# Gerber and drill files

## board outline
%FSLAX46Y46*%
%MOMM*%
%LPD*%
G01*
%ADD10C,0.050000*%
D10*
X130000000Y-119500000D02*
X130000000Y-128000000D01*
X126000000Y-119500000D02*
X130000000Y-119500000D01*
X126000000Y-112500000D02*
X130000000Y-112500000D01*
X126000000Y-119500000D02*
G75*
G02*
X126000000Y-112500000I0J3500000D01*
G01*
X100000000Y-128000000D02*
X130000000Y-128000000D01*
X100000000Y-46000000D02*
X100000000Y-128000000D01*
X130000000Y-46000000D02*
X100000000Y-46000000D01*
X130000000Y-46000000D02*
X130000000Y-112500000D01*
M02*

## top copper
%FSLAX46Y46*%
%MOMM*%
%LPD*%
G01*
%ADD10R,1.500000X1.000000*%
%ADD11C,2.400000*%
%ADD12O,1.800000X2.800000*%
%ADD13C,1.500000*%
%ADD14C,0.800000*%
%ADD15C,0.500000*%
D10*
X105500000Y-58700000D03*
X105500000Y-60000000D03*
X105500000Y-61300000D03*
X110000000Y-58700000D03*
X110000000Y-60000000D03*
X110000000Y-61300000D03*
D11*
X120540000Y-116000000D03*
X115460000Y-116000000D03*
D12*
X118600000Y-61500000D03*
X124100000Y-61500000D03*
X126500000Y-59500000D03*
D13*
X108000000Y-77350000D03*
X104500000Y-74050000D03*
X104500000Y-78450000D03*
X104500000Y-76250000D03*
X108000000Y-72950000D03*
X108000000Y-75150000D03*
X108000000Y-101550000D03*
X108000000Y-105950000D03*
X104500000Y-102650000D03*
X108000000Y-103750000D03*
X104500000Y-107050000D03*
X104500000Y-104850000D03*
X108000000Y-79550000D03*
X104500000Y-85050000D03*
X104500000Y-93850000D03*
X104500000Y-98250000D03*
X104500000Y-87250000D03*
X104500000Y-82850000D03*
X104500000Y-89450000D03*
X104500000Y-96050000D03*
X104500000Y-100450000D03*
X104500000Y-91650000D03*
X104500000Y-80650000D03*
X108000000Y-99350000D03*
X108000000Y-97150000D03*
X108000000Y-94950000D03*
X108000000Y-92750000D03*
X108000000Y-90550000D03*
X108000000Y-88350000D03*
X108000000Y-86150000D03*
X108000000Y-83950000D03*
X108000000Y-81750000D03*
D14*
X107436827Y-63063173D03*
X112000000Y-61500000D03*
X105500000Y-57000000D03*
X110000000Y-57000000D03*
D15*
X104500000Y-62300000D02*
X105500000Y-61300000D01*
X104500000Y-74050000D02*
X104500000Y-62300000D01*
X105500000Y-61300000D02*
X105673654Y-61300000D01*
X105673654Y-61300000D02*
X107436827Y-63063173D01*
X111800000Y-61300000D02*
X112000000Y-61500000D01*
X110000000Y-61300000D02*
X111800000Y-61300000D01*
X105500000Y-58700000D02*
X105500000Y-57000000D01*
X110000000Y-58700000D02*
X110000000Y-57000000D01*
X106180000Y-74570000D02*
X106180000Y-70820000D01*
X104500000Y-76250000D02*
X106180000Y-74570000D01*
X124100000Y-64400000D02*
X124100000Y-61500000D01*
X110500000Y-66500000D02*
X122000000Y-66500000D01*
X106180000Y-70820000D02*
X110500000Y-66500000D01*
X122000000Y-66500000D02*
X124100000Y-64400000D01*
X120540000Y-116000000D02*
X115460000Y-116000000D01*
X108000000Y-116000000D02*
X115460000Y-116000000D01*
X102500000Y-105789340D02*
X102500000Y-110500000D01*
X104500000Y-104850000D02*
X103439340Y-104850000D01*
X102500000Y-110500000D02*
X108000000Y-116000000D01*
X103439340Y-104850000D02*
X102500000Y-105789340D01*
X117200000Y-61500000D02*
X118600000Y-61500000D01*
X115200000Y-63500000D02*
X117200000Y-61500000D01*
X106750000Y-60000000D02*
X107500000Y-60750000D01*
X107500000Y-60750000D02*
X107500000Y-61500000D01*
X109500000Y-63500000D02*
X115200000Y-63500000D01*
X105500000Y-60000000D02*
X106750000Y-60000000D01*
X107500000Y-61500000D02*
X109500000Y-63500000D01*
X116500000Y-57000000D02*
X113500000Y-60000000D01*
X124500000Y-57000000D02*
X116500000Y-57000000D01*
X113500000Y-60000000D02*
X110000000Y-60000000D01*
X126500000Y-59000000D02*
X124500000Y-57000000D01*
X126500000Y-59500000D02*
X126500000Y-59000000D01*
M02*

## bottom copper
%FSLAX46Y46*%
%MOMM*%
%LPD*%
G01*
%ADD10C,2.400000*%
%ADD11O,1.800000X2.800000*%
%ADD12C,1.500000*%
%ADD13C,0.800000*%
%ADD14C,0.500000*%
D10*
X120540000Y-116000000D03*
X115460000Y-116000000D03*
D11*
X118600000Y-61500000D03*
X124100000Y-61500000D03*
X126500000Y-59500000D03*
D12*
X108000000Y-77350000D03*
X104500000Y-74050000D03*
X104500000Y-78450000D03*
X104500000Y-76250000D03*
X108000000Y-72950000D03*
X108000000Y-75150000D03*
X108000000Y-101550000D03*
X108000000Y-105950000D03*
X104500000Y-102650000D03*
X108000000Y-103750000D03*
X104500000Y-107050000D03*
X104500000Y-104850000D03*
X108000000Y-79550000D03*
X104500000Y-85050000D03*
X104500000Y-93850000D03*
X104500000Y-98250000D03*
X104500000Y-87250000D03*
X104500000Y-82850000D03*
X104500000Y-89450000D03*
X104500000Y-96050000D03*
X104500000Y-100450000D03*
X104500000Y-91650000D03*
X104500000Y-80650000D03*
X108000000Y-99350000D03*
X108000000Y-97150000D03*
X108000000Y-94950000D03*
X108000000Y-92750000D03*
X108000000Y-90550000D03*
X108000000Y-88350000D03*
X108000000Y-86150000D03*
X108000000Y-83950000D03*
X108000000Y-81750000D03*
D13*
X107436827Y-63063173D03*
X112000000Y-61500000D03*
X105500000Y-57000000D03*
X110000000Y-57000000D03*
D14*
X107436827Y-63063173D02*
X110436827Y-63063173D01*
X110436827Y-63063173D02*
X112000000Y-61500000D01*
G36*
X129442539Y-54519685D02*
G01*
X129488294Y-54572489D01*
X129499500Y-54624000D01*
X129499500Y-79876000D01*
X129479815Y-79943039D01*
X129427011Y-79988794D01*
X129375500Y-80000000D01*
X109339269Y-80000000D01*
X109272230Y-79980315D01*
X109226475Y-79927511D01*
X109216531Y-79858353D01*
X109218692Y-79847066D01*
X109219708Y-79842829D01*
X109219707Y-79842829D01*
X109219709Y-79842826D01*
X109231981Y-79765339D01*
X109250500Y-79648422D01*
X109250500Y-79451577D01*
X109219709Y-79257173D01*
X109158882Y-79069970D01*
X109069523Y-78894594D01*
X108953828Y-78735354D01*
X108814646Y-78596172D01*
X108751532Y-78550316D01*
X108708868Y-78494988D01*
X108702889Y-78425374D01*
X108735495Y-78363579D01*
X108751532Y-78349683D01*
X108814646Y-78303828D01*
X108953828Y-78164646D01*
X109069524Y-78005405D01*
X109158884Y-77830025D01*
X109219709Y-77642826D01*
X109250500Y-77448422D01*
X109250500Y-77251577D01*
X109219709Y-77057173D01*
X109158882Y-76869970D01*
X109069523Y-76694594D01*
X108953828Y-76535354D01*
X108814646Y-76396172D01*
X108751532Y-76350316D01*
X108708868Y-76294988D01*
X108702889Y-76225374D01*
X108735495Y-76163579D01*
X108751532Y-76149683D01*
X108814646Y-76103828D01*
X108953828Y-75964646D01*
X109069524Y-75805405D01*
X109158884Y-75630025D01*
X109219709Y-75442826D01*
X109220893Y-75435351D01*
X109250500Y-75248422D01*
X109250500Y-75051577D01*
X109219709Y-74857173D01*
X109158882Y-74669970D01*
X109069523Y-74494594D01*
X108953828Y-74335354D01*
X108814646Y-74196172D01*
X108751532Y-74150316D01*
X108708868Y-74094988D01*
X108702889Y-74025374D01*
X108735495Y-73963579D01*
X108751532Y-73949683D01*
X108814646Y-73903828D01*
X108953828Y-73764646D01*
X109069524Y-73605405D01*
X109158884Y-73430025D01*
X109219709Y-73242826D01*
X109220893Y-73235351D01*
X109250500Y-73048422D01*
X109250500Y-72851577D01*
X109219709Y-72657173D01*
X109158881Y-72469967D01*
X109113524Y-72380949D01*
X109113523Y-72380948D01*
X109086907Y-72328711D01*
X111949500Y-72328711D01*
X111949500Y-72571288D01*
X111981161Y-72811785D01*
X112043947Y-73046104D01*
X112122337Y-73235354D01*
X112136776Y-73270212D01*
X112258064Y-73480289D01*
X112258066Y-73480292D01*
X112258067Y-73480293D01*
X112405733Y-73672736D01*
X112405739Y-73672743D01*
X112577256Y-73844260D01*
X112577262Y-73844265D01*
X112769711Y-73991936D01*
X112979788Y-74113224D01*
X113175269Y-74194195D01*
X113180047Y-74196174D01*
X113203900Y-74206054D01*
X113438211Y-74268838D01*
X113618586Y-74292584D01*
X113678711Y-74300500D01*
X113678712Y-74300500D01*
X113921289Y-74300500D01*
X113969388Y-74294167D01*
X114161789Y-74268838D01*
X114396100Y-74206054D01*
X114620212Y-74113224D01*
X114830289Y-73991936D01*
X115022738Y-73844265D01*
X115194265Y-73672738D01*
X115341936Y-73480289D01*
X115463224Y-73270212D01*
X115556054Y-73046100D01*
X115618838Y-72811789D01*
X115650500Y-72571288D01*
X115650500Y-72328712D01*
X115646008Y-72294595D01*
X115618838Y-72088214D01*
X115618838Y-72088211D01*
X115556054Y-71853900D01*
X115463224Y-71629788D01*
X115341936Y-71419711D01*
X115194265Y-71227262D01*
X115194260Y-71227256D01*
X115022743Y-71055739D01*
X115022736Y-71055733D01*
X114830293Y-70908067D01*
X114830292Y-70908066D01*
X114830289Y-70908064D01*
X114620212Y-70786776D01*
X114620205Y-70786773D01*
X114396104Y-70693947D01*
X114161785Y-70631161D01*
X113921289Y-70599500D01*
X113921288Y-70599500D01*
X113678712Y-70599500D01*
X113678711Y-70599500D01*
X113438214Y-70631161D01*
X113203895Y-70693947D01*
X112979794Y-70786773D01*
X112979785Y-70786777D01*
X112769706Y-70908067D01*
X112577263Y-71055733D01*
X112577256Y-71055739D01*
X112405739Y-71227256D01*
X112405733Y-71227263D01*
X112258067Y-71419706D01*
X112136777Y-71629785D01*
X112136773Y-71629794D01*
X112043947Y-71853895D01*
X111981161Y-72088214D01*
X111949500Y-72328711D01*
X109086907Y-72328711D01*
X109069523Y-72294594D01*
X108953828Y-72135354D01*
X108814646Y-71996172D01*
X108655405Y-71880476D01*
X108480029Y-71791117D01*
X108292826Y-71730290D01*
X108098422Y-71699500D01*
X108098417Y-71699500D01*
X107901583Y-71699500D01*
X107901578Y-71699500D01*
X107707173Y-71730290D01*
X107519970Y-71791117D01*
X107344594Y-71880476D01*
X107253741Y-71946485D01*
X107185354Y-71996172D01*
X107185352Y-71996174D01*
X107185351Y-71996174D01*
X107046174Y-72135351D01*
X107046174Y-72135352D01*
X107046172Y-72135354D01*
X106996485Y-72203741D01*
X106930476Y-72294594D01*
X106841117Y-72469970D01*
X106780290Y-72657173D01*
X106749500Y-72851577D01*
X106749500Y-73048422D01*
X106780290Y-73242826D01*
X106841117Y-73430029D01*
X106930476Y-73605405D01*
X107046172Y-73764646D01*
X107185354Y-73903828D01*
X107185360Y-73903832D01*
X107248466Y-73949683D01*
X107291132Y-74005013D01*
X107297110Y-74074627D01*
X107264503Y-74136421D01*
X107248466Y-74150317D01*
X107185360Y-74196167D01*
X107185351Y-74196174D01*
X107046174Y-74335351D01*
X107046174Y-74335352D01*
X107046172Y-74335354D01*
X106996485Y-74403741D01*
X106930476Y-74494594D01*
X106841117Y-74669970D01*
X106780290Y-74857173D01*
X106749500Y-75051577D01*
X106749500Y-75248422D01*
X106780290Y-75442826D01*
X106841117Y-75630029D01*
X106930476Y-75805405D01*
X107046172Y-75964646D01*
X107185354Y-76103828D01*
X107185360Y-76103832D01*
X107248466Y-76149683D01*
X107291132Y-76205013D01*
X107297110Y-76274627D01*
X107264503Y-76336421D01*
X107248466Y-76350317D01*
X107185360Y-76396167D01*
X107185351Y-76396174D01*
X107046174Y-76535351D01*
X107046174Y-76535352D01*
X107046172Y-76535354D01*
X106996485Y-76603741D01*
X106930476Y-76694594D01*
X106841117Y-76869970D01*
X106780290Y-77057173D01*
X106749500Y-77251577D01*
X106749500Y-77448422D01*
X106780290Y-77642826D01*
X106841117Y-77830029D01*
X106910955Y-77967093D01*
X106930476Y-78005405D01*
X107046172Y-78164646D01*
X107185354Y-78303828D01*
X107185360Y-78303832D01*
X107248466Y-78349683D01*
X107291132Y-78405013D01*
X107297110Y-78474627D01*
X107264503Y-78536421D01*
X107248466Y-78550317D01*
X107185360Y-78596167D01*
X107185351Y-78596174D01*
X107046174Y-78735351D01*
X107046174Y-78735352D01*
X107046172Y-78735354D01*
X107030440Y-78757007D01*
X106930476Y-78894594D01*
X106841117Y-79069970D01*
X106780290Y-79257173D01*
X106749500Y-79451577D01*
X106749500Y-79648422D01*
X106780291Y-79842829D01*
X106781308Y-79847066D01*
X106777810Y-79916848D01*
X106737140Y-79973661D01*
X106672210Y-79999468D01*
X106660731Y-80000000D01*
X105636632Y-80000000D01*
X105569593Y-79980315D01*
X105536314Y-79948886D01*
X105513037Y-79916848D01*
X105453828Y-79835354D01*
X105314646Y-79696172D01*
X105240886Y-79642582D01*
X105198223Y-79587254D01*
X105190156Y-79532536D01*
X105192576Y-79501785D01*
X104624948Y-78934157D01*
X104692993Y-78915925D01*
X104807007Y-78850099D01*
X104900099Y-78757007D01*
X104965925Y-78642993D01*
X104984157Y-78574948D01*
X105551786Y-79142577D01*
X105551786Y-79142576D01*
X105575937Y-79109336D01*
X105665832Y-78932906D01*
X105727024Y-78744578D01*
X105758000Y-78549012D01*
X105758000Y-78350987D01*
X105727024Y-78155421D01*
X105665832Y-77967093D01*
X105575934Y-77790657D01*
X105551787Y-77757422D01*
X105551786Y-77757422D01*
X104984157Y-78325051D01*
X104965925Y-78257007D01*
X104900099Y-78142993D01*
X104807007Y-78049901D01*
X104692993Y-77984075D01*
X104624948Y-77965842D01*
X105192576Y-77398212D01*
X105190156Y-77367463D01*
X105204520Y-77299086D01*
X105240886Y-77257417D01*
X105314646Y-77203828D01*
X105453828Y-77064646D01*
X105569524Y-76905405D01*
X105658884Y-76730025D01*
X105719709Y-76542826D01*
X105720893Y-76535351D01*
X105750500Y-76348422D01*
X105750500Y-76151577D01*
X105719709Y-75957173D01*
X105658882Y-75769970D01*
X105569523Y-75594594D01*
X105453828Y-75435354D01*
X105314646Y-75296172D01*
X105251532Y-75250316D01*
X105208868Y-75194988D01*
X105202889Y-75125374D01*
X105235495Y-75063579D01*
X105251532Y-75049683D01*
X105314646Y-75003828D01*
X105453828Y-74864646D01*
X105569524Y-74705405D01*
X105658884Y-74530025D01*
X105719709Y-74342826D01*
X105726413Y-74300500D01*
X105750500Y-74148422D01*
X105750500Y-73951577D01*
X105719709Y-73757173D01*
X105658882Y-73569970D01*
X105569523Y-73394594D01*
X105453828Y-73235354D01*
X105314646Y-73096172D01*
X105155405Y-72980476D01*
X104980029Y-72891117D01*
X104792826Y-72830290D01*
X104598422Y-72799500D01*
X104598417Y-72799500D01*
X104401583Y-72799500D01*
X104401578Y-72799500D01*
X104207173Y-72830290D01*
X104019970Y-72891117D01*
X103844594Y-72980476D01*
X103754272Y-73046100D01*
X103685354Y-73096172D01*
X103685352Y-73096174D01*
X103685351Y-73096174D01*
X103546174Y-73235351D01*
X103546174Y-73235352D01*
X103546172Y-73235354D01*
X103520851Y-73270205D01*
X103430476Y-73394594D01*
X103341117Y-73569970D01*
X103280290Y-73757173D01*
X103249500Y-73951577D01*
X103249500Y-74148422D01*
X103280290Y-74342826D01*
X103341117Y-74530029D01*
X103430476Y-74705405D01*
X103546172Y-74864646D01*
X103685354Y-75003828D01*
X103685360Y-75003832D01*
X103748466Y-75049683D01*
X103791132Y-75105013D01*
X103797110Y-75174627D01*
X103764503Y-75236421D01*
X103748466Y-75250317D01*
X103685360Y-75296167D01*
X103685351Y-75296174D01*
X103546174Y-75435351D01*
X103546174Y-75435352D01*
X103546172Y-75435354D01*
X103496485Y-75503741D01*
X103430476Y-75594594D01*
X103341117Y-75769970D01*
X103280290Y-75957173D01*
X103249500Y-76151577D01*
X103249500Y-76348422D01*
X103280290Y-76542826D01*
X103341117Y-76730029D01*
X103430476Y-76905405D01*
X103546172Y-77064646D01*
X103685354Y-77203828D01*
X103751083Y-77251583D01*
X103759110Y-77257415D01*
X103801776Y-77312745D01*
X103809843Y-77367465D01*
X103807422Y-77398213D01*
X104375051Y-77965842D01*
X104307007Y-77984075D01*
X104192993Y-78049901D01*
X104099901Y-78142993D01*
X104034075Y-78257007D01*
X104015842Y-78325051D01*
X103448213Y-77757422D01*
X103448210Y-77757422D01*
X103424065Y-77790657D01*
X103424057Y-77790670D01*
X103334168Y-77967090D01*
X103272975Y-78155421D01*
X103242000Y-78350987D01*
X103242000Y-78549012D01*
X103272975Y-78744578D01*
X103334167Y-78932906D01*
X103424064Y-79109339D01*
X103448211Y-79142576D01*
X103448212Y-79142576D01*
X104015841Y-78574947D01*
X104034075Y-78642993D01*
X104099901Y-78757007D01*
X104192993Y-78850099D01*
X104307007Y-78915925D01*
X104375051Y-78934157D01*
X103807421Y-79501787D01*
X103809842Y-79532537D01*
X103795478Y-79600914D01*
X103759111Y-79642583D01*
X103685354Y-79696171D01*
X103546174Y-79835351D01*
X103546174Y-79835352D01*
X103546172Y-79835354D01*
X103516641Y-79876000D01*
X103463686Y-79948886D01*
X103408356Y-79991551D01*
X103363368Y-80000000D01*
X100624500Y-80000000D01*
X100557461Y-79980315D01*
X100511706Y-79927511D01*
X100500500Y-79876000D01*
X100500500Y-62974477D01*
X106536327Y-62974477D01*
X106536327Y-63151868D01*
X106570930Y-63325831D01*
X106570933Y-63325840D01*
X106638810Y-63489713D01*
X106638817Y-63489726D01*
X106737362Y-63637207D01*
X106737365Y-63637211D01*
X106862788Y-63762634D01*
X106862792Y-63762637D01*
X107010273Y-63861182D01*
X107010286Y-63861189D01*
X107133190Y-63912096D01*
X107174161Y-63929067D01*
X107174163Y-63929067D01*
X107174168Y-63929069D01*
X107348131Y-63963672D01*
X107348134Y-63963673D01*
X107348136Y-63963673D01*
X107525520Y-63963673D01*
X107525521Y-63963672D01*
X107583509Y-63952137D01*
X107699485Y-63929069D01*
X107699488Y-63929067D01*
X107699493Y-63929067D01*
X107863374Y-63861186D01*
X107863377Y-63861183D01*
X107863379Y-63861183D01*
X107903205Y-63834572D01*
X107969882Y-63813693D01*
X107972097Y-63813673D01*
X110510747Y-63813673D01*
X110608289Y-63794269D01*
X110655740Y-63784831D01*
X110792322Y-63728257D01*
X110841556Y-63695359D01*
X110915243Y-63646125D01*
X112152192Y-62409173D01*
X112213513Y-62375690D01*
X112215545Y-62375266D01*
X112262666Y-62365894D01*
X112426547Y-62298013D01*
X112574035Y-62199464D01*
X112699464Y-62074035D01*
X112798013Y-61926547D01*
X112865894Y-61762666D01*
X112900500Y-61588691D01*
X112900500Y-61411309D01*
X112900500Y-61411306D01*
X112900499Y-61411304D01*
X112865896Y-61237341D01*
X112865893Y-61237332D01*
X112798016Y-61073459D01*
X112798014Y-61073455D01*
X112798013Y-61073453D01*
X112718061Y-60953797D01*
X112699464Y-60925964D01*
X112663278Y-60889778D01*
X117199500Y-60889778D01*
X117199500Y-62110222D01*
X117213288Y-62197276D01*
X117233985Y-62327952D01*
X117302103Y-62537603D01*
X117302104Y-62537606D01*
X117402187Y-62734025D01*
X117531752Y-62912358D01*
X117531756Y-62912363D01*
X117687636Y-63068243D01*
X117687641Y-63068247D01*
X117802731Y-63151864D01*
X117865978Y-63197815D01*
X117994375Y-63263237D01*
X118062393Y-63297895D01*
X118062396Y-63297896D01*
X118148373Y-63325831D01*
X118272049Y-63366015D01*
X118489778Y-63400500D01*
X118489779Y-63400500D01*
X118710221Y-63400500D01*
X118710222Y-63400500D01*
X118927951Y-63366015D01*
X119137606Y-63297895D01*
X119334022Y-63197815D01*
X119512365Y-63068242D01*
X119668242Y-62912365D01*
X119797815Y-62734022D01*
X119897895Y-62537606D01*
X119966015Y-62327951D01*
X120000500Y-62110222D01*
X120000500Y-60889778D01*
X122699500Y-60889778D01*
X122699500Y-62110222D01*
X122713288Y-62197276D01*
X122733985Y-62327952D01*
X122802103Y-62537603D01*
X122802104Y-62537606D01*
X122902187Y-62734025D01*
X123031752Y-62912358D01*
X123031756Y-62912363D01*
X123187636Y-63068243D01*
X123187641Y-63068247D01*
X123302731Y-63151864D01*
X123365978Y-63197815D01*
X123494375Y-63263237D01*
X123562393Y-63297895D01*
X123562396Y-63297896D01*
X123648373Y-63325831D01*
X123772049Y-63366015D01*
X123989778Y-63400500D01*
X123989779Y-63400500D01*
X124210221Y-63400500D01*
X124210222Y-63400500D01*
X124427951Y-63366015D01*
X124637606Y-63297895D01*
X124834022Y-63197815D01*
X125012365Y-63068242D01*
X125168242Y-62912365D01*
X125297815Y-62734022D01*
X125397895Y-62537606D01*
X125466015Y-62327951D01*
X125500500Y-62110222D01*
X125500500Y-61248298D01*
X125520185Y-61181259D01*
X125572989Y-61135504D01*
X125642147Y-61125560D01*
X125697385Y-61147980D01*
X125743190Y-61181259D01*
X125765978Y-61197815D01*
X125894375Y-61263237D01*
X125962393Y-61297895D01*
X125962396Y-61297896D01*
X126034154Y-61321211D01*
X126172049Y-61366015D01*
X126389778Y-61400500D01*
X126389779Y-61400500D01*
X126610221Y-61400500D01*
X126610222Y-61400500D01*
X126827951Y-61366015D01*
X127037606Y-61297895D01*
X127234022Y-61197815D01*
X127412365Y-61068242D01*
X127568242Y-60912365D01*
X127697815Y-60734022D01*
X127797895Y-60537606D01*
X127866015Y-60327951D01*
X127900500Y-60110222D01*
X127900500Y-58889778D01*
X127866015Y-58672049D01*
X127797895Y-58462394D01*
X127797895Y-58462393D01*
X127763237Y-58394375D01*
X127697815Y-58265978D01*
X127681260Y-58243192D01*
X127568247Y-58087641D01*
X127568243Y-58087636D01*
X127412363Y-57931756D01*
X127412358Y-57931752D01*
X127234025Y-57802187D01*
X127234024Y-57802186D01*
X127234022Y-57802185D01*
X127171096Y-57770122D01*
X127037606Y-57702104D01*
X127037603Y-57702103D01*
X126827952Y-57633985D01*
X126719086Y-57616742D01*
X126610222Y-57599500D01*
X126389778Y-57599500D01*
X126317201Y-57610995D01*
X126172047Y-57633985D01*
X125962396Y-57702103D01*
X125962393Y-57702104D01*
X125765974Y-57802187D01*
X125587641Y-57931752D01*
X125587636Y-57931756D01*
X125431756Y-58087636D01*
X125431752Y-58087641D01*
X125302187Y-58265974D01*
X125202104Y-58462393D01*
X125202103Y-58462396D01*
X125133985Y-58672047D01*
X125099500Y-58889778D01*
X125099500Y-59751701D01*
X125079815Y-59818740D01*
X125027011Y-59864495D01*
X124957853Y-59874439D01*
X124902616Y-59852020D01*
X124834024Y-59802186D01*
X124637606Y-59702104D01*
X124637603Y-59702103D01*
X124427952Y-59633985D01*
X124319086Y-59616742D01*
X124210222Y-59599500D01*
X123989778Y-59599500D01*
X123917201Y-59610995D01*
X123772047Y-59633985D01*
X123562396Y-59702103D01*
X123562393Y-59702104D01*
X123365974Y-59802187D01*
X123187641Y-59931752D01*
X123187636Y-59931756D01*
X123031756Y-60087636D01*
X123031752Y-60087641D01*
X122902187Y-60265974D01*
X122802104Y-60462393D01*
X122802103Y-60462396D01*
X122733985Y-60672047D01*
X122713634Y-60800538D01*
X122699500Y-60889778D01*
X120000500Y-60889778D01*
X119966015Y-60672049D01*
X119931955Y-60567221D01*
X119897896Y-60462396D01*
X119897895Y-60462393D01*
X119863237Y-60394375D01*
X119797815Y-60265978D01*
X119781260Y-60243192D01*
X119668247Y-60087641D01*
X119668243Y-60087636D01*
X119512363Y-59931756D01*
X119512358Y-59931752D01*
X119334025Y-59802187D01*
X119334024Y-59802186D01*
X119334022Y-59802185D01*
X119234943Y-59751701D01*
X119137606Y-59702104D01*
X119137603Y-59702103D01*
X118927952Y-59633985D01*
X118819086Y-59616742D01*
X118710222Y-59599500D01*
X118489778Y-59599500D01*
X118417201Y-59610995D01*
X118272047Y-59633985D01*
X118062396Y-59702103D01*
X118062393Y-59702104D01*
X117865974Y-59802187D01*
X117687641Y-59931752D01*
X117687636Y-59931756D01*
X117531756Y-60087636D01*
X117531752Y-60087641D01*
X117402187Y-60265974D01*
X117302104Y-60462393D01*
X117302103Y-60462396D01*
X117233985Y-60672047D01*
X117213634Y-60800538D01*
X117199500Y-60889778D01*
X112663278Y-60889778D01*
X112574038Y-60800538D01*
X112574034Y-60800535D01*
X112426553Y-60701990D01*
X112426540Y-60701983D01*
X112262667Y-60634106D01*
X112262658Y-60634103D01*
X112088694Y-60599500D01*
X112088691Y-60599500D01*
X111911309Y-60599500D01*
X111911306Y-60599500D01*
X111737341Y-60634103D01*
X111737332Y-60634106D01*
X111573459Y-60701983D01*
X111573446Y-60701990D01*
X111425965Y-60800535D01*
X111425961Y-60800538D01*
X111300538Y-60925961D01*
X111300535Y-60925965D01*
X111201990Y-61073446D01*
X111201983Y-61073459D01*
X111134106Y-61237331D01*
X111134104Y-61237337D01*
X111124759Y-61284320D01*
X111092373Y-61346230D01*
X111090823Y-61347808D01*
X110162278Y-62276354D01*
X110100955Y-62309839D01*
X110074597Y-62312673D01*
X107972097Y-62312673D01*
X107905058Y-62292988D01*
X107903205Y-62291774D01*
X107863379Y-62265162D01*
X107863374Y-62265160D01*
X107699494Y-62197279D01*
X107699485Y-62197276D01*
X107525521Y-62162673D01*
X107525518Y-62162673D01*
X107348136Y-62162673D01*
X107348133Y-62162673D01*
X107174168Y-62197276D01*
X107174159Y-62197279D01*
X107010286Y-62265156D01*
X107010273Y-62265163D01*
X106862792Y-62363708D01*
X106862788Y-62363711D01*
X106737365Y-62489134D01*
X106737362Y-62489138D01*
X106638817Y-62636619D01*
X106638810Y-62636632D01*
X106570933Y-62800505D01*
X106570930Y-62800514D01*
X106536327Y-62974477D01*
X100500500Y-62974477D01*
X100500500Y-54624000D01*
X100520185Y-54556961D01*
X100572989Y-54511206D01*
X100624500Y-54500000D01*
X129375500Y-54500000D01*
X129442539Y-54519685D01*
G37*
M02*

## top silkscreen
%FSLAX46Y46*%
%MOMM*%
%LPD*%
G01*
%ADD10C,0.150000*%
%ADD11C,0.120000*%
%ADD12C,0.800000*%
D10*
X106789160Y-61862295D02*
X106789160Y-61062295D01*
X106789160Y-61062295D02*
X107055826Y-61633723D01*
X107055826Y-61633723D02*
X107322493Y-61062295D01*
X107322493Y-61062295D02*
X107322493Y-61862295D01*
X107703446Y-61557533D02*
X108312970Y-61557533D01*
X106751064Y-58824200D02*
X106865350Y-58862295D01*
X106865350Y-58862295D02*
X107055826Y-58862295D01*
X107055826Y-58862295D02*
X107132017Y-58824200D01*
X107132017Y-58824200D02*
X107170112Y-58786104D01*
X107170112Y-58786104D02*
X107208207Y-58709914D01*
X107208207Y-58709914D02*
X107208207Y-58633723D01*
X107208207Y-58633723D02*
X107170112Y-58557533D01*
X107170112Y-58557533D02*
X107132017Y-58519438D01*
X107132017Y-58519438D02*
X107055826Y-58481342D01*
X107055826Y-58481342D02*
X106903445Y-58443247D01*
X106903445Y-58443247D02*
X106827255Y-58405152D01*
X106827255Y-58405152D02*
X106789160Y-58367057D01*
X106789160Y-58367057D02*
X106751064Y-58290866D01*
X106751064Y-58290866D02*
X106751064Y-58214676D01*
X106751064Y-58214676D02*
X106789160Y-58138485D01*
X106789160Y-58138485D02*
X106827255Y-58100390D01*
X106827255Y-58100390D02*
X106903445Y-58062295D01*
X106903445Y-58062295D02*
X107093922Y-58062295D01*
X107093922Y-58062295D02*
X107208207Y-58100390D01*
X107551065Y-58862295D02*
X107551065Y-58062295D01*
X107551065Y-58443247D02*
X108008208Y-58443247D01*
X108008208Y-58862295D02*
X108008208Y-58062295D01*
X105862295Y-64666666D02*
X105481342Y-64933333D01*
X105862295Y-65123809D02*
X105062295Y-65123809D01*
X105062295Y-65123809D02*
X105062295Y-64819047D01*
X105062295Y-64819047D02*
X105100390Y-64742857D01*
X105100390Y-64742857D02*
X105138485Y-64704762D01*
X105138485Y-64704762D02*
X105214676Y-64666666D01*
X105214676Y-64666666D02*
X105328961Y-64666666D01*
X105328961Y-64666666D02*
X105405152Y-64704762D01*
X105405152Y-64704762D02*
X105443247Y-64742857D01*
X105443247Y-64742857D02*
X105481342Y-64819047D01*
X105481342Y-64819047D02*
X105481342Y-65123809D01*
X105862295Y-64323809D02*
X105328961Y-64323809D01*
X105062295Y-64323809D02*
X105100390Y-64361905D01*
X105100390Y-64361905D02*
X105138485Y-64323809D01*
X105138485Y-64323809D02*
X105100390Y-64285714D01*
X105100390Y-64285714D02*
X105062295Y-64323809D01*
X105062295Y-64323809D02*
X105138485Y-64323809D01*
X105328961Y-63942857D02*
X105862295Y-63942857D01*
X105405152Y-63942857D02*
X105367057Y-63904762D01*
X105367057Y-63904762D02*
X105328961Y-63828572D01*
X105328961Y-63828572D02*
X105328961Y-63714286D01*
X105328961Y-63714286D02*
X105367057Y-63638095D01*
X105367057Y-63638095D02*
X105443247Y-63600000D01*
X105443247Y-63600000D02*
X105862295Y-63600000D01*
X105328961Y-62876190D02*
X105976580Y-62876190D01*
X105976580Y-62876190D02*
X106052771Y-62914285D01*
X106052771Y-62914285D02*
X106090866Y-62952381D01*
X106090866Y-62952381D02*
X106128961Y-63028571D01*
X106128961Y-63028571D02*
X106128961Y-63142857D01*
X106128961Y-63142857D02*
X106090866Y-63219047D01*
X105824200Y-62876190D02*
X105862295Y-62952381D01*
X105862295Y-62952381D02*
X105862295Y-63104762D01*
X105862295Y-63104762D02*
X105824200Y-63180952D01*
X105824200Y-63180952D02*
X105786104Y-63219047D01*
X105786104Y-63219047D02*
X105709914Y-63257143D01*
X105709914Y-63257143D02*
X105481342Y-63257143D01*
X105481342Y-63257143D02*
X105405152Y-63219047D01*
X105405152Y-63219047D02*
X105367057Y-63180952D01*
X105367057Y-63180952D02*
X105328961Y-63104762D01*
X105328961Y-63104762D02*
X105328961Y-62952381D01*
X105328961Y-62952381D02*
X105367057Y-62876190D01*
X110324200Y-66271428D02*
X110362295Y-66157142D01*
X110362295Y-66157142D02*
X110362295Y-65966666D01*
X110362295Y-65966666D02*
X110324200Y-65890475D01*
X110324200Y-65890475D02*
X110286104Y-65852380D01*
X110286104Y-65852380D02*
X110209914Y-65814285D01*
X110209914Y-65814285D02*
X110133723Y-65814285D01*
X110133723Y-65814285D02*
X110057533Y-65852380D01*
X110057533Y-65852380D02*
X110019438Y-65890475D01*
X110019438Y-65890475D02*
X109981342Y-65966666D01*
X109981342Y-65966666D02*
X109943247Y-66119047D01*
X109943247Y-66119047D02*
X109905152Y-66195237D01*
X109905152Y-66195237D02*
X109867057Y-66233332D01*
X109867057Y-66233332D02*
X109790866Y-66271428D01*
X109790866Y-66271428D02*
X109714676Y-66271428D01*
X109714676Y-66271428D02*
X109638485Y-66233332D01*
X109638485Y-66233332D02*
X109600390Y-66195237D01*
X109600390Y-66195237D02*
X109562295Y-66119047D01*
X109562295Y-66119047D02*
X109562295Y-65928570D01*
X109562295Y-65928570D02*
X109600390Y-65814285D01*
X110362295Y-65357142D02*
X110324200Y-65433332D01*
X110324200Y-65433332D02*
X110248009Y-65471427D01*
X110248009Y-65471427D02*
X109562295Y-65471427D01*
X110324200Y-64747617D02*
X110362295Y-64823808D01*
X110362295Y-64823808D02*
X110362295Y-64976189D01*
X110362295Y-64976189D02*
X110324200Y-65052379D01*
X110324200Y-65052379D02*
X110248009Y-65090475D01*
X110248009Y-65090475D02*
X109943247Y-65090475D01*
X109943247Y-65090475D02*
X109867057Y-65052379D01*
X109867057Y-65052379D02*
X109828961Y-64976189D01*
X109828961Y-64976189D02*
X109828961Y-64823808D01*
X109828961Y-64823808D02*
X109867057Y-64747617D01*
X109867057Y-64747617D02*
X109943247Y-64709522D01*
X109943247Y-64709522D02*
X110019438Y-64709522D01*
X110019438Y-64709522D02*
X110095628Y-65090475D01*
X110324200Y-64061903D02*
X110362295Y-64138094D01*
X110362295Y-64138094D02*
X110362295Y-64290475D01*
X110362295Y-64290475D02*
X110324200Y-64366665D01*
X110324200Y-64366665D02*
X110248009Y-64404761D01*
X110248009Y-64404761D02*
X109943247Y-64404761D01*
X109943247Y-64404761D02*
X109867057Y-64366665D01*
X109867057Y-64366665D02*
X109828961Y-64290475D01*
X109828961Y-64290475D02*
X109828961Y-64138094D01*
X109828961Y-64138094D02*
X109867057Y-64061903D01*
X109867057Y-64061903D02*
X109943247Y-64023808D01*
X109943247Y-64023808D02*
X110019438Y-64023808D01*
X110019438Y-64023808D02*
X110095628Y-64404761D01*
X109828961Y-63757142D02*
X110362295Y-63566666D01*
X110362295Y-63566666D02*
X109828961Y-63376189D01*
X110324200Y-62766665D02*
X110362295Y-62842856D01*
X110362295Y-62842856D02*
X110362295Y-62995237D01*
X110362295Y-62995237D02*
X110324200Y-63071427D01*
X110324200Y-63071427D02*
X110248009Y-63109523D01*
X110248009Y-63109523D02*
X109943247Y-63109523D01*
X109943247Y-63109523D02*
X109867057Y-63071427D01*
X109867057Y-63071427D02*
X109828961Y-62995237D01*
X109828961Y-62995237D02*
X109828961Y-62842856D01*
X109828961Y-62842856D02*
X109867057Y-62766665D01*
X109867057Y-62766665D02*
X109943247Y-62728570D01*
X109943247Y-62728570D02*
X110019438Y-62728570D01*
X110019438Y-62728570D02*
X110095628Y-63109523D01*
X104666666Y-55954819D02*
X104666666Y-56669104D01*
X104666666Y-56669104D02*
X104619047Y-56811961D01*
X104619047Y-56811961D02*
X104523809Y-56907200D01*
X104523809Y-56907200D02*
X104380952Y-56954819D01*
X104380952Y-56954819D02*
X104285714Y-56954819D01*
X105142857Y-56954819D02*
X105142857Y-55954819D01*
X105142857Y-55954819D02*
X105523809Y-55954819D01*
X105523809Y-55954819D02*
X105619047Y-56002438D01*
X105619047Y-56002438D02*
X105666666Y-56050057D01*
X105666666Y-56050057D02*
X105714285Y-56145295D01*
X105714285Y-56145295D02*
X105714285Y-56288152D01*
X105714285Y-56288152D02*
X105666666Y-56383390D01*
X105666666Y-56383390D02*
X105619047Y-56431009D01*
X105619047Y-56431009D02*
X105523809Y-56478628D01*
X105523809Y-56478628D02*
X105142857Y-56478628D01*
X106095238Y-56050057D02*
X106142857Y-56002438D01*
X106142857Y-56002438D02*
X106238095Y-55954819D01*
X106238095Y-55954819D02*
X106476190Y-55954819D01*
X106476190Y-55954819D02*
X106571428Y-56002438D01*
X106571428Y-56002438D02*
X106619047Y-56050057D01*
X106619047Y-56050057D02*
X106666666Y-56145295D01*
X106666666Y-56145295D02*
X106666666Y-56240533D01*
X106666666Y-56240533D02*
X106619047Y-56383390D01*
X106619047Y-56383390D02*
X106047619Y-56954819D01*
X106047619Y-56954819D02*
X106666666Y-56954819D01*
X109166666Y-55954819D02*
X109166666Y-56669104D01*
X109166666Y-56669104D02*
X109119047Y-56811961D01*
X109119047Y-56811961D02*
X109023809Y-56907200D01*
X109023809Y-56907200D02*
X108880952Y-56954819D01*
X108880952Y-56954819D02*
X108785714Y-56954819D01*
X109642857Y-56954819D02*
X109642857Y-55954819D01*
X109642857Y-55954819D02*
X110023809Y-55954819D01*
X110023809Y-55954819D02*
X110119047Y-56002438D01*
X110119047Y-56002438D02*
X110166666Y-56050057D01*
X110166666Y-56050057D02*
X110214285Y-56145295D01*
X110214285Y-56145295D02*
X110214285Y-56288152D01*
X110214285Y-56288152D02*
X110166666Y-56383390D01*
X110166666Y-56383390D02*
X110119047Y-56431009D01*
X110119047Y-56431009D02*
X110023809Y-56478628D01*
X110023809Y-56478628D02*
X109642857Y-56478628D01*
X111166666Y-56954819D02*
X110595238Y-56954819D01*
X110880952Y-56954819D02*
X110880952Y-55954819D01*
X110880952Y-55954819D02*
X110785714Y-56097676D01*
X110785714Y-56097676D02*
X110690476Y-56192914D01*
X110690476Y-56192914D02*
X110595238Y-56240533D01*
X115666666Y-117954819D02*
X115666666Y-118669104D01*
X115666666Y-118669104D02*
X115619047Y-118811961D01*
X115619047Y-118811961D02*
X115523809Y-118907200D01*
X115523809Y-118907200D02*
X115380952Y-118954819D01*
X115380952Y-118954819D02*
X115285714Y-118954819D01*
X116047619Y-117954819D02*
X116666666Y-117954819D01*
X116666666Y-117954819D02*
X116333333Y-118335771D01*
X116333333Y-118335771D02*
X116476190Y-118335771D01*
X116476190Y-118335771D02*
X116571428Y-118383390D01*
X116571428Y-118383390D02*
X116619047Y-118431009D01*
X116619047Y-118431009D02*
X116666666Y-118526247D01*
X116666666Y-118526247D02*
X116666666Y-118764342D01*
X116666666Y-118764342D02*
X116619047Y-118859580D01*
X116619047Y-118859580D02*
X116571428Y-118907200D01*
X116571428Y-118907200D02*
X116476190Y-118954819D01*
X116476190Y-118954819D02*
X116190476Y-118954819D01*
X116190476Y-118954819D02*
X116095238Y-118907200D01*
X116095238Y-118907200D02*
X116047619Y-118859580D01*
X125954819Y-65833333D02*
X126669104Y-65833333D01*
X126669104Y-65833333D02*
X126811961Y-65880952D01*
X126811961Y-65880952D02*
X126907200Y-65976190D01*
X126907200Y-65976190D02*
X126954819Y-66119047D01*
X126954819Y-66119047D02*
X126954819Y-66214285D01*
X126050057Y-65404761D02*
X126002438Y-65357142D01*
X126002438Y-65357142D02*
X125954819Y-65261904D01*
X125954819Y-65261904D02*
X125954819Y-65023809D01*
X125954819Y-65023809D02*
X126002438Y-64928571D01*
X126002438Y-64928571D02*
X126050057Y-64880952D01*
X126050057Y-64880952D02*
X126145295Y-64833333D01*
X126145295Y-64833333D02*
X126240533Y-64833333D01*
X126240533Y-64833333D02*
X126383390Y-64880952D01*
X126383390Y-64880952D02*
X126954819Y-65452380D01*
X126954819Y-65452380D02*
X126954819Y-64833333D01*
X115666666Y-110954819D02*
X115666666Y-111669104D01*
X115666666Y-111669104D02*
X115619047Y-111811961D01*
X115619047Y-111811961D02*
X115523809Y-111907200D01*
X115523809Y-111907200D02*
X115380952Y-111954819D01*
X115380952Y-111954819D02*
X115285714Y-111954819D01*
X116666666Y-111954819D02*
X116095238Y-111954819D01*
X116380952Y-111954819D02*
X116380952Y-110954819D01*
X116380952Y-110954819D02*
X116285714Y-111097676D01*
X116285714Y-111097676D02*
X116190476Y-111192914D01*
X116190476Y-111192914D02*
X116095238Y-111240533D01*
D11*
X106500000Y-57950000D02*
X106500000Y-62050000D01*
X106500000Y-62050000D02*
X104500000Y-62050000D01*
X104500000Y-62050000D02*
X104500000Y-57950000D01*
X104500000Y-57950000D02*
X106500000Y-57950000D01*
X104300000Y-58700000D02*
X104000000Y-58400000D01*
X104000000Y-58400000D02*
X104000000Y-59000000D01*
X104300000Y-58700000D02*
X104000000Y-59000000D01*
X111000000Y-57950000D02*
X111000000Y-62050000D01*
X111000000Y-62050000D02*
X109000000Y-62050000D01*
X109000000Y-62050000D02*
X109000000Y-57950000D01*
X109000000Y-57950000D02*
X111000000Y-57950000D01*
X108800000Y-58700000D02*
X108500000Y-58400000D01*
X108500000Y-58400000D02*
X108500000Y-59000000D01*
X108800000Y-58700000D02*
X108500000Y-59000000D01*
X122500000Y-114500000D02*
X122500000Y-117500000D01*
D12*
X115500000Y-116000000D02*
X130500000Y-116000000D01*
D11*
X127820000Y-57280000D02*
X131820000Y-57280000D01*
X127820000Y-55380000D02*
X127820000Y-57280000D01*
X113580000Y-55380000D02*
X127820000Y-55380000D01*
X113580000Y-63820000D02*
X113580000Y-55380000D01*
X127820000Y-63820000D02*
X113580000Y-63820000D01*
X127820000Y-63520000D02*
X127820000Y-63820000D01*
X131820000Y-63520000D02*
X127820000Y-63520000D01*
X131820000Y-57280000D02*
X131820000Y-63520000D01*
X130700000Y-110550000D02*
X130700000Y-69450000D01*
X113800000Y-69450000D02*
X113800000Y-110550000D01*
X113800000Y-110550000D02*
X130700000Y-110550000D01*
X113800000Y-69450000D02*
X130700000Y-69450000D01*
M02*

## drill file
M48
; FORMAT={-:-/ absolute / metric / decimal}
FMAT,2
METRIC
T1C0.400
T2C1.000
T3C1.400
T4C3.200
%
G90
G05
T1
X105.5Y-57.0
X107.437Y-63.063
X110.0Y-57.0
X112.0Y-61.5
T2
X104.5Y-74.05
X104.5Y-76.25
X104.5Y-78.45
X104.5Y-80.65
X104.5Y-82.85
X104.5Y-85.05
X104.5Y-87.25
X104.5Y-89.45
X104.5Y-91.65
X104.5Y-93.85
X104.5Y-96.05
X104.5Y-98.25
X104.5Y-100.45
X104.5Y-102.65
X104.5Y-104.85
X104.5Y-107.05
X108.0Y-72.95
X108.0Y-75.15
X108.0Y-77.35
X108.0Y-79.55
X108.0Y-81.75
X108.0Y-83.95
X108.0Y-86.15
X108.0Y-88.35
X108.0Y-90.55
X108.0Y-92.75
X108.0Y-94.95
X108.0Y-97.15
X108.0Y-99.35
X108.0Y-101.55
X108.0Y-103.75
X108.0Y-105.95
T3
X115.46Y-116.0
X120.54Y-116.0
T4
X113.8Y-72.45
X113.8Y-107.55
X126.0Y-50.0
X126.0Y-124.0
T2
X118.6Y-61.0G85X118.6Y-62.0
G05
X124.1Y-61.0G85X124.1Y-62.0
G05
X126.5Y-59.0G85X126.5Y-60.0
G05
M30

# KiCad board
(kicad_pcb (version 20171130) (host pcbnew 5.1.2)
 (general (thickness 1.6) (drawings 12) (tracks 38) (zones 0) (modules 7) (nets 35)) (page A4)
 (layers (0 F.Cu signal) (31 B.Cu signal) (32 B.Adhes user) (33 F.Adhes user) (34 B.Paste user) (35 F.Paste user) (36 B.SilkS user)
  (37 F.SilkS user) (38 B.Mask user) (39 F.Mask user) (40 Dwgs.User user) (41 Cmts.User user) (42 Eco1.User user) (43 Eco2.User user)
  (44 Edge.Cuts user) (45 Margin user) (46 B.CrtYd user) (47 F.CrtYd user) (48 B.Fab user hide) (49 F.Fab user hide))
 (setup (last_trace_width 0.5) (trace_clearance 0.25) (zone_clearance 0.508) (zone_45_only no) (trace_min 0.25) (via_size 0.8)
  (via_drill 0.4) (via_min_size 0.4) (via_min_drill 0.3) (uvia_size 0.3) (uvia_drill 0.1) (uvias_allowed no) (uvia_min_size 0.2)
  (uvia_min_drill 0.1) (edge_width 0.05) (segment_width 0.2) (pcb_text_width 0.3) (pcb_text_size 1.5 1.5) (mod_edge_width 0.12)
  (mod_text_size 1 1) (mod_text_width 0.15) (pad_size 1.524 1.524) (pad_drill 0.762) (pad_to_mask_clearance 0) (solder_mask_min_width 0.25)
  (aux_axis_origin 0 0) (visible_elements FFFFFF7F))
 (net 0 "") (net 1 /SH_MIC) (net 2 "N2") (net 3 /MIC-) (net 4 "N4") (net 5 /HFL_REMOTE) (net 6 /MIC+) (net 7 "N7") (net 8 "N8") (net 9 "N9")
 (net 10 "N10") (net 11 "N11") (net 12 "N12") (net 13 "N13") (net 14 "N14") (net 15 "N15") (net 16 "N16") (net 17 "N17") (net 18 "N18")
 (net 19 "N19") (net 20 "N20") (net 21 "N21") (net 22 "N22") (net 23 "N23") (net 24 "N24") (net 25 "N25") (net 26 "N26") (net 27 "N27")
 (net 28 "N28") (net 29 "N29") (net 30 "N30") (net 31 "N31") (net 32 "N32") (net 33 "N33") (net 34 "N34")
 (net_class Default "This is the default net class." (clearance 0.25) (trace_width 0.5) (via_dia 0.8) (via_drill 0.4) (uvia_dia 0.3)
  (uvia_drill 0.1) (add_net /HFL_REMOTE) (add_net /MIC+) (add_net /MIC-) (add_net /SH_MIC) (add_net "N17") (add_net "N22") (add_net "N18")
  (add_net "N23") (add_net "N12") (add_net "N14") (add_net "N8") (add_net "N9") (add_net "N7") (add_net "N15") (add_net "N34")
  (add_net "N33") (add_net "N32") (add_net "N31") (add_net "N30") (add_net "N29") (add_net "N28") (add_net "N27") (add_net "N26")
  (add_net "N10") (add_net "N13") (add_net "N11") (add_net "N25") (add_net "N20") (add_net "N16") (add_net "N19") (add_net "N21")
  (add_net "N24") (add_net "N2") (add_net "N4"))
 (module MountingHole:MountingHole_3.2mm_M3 (layer F.Cu) (at 126 124)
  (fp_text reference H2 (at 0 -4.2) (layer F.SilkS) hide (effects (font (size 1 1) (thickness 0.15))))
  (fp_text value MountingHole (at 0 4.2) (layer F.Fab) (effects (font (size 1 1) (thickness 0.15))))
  (pad 1 np_thru_hole circle (at 0 0) (size 3.2 3.2) (drill 3.2) (layers *.Cu *.Mask)))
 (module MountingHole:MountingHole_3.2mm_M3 (layer F.Cu) (at 126 50)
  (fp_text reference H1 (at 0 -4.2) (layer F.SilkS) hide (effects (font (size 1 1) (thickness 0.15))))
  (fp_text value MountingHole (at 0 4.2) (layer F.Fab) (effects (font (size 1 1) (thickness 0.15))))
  (pad 1 np_thru_hole circle (at 0 0) (size 3.2 3.2) (drill 3.2) (layers *.Cu *.Mask)))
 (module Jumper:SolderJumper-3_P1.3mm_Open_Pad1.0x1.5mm (layer F.Cu) (at 105.5 60 270)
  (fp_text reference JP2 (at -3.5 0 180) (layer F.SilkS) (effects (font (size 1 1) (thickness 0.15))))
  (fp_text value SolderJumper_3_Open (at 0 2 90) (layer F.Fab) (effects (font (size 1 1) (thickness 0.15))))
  (fp_line (start -2.05 -1) (end 2.05 -1) (layer F.SilkS) (width 0.12))
  (fp_line (start 2.05 -1) (end 2.05 1) (layer F.SilkS) (width 0.12))
  (fp_line (start 2.05 1) (end -2.05 1) (layer F.SilkS) (width 0.12))
  (fp_line (start -2.05 1) (end -2.05 -1) (layer F.SilkS) (width 0.12))
  (fp_line (start -1.3 1.2) (end -1.6 1.5) (layer F.SilkS) (width 0.12))
  (fp_line (start -1.6 1.5) (end -1 1.5) (layer F.SilkS) (width 0.12))
  (fp_line (start -1.3 1.2) (end -1 1.5) (layer F.SilkS) (width 0.12))
  (pad 1 smd rect (at -1.3 0 270) (size 1 1.5) (layers F.Cu F.Mask) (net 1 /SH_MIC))
  (pad 2 smd rect (at 0 0 270) (size 1 1.5) (layers F.Cu F.Mask) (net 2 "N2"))
  (pad 3 smd rect (at 1.3 0 270) (size 1 1.5) (layers F.Cu F.Mask) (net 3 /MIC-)))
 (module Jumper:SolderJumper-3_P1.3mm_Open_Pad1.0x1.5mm (layer F.Cu) (at 110 60 270)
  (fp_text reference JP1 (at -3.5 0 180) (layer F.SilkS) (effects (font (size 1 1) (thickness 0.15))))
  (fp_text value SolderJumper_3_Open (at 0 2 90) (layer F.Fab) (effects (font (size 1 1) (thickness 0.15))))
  (fp_line (start -2.05 -1) (end 2.05 -1) (layer F.SilkS) (width 0.12))
  (fp_line (start 2.05 -1) (end 2.05 1) (layer F.SilkS) (width 0.12))
  (fp_line (start 2.05 1) (end -2.05 1) (layer F.SilkS) (width 0.12))
  (fp_line (start -2.05 1) (end -2.05 -1) (layer F.SilkS) (width 0.12))
  (fp_line (start -1.3 1.2) (end -1.6 1.5) (layer F.SilkS) (width 0.12))
  (fp_line (start -1.6 1.5) (end -1 1.5) (layer F.SilkS) (width 0.12))
  (fp_line (start -1.3 1.2) (end -1 1.5) (layer F.SilkS) (width 0.12))
  (pad 1 smd rect (at -1.3 0 270) (size 1 1.5) (layers F.Cu F.Mask) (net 1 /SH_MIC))
  (pad 2 smd rect (at 0 0 270) (size 1 1.5) (layers F.Cu F.Mask) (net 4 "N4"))
  (pad 3 smd rect (at 1.3 0 270) (size 1 1.5) (layers F.Cu F.Mask) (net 3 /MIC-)))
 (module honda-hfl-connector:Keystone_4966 (layer F.Cu) (at 118 116)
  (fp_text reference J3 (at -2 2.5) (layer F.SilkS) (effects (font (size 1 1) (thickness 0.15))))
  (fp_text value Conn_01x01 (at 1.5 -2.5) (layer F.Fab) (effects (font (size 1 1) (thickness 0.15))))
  (fp_line (start 4.5 -1.5) (end 4.5 1.5) (layer F.SilkS) (width 0.12))
  (fp_line (start -2.5 0) (end 12.5 0) (layer F.SilkS) (width 0.8))
  (pad 1 thru_hole circle (at 2.54 0) (size 2.4 2.4) (drill 1.4) (layers *.Cu *.Mask) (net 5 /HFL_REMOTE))
  (pad 1 thru_hole circle (at -2.54 0) (size 2.4 2.4) (drill 1.4) (layers *.Cu *.Mask) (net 5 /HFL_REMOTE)))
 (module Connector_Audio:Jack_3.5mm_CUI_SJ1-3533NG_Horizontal (layer F.Cu) (at 126.5 59.5 270)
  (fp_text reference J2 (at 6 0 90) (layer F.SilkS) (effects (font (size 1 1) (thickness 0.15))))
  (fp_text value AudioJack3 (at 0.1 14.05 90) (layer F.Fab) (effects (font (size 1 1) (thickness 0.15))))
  (fp_line (start -2.22 -1.32) (end -2.22 -5.32) (layer F.SilkS) (width 0.12))
  (fp_line (start -4.12 -1.32) (end -2.22 -1.32) (layer F.SilkS) (width 0.12))
  (fp_line (start -4.12 12.92) (end -4.12 -1.32) (layer F.SilkS) (width 0.12))
  (fp_line (start 4.32 12.92) (end -4.12 12.92) (layer F.SilkS) (width 0.12))
  (fp_line (start 4.32 -1.32) (end 4.32 12.92) (layer F.SilkS) (width 0.12))
  (fp_line (start 4.02 -1.32) (end 4.32 -1.32) (layer F.SilkS) (width 0.12))
  (fp_line (start 4.02 -5.32) (end 4.02 -1.32) (layer F.SilkS) (width 0.12))
  (fp_line (start -2.22 -5.32) (end 4.02 -5.32) (layer F.SilkS) (width 0.12))
  (pad R thru_hole oval (at 2 7.9 270) (size 2.8 1.8) (drill oval 2 1) (layers *.Cu *.Mask) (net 2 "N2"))
  (pad T thru_hole oval (at 2 2.4 270) (size 2.8 1.8) (drill oval 2 1) (layers *.Cu *.Mask) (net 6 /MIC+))
  (pad S thru_hole oval (at 0 0 270) (size 2.8 1.8) (drill oval 2 1) (layers *.Cu *.Mask) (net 4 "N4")))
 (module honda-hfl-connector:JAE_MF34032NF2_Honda (layer F.Cu) (at 108 90)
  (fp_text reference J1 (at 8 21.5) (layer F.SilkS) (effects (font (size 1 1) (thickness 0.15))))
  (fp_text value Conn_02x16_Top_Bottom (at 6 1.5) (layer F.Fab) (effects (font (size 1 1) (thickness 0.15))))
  (fp_line (start 22.7 20.55) (end 22.7 -20.55) (layer F.SilkS) (width 0.12))
  (fp_line (start 5.8 -20.55) (end 5.8 20.55) (layer F.SilkS) (width 0.12))
  (fp_line (start 5.8 20.55) (end 22.7 20.55) (layer F.SilkS) (width 0.12))
  (fp_line (start 5.8 -20.55) (end 22.7 -20.55) (layer F.SilkS) (width 0.12))
  (pad 19 thru_hole circle (at 0 -12.65) (size 1.5 1.5) (drill 1) (layers *.Cu *.Mask) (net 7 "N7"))
  (pad 1 thru_hole circle (at -3.5 -15.95) (size 1.5 1.5) (drill 1) (layers *.Cu *.Mask) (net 3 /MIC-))
  (pad 3 thru_hole circle (at -3.5 -11.55) (size 1.5 1.5) (drill 1) (layers *.Cu *.Mask) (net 1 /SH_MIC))
  (pad 2 thru_hole circle (at -3.5 -13.75) (size 1.5 1.5) (drill 1) (layers *.Cu *.Mask) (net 6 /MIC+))
  (pad 17 thru_hole circle (at 0 -17.05) (size 1.5 1.5) (drill 1) (layers *.Cu *.Mask) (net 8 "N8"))
  (pad 18 thru_hole circle (at 0 -14.85) (size 1.5 1.5) (drill 1) (layers *.Cu *.Mask) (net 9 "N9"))
  (pad 30 thru_hole circle (at 0 11.55) (size 1.5 1.5) (drill 1) (layers *.Cu *.Mask) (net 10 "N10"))
  (pad 32 thru_hole circle (at 0 15.95) (size 1.5 1.5) (drill 1) (layers *.Cu *.Mask) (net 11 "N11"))
  (pad 14 thru_hole circle (at -3.5 12.65) (size 1.5 1.5) (drill 1) (layers *.Cu *.Mask) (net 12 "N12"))
  (pad 31 thru_hole circle (at 0 13.75) (size 1.5 1.5) (drill 1) (layers *.Cu *.Mask) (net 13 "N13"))
  (pad 16 thru_hole circle (at -3.5 17.05) (size 1.5 1.5) (drill 1) (layers *.Cu *.Mask) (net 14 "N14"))
  (pad 15 thru_hole circle (at -3.5 14.85) (size 1.5 1.5) (drill 1) (layers *.Cu *.Mask) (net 5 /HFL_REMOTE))
  (pad 20 thru_hole circle (at 0 -10.45) (size 1.5 1.5) (drill 1) (layers *.Cu *.Mask) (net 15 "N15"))
  (pad "" np_thru_hole circle (at 5.8 17.55) (size 3.2 3.2) (drill 3.2) (layers *.Cu *.Mask))
  (pad 6 thru_hole circle (at -3.5 -4.95) (size 1.5 1.5) (drill 1) (layers *.Cu *.Mask) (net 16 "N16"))
  (pad 10 thru_hole circle (at -3.5 3.85) (size 1.5 1.5) (drill 1) (layers *.Cu *.Mask) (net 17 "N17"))
  (pad 12 thru_hole circle (at -3.5 8.25) (size 1.5 1.5) (drill 1) (layers *.Cu *.Mask) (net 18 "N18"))
  (pad 7 thru_hole circle (at -3.5 -2.75) (size 1.5 1.5) (drill 1) (layers *.Cu *.Mask) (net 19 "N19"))
  (pad 5 thru_hole circle (at -3.5 -7.15) (size 1.5 1.5) (drill 1) (layers *.Cu *.Mask) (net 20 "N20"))
  (pad 8 thru_hole circle (at -3.5 -0.55) (size 1.5 1.5) (drill 1) (layers *.Cu *.Mask) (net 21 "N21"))
  (pad 11 thru_hole circle (at -3.5 6.05) (size 1.5 1.5) (drill 1) (layers *.Cu *.Mask) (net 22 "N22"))
  (pad 13 thru_hole circle (at -3.5 10.45) (size 1.5 1.5) (drill 1) (layers *.Cu *.Mask) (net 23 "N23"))
  (pad 9 thru_hole circle (at -3.5 1.65) (size 1.5 1.5) (drill 1) (layers *.Cu *.Mask) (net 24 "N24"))
  (pad 4 thru_hole circle (at -3.5 -9.35) (size 1.5 1.5) (drill 1) (layers *.Cu *.Mask) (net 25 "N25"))
  (pad 29 thru_hole circle (at 0 9.35) (size 1.5 1.5) (drill 1) (layers *.Cu *.Mask) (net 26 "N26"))
  (pad 28 thru_hole circle (at 0 7.15) (size 1.5 1.5) (drill 1) (layers *.Cu *.Mask) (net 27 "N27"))
  (pad 27 thru_hole circle (at 0 4.95) (size 1.5 1.5) (drill 1) (layers *.Cu *.Mask) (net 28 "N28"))
  (pad 26 thru_hole circle (at 0 2.75) (size 1.5 1.5) (drill 1) (layers *.Cu *.Mask) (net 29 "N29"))
  (pad 25 thru_hole circle (at 0 0.55) (size 1.5 1.5) (drill 1) (layers *.Cu *.Mask) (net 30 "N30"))
  (pad 24 thru_hole circle (at 0 -1.65) (size 1.5 1.5) (drill 1) (layers *.Cu *.Mask) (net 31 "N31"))
  (pad 23 thru_hole circle (at 0 -3.85) (size 1.5 1.5) (drill 1) (layers *.Cu *.Mask) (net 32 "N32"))
  (pad 22 thru_hole circle (at 0 -6.05) (size 1.5 1.5) (drill 1) (layers *.Cu *.Mask) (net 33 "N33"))
  (pad 21 thru_hole circle (at 0 -8.25) (size 1.5 1.5) (drill 1) (layers *.Cu *.Mask) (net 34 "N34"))
  (pad "" np_thru_hole circle (at 5.8 -17.55) (size 3.2 3.2) (drill 3.2) (layers *.Cu *.Mask)))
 (gr_line (start 130 119.5) (end 130 128) (layer Edge.Cuts) (width 0.05))
 (gr_line (start 126 119.5) (end 130 119.5) (layer Edge.Cuts) (width 0.05))
 (gr_line (start 126 112.5) (end 130 112.5) (layer Edge.Cuts) (width 0.05))
 (gr_arc (start 126 116) (end 126 112.5) (angle -180) (layer Edge.Cuts) (width 0.05))
 (gr_line (start 100 128) (end 130 128) (layer Edge.Cuts) (width 0.05))
 (gr_line (start 100 46) (end 100 128) (layer Edge.Cuts) (width 0.05))
 (gr_line (start 130 46) (end 100 46) (layer Edge.Cuts) (width 0.05))
 (gr_line (start 130 46) (end 130 112.5) (layer Edge.Cuts) (width 0.05))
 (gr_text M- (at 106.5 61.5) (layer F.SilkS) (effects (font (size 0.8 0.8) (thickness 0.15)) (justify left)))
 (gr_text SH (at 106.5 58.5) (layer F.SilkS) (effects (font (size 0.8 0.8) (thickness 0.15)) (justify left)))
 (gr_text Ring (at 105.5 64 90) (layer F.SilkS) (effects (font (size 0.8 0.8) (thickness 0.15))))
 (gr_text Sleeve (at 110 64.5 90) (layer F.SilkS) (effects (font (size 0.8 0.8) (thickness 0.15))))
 (segment (start 104.5 62.3) (end 105.5 61.3) (width 0.5) (layer F.Cu) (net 3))
 (segment (start 104.5 74.05) (end 104.5 62.3) (width 0.5) (layer F.Cu) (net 3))
 (segment (start 105.5 61.3) (end 105.673654 61.3) (width 0.5) (layer F.Cu) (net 3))
 (via (at 107.436827 63.063173) (size 0.8) (drill 0.4) (layers F.Cu B.Cu) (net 3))
 (segment (start 105.673654 61.3) (end 107.436827 63.063173) (width 0.5) (layer F.Cu) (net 3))
 (via (at 112 61.5) (size 0.8) (drill 0.4) (layers F.Cu B.Cu) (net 3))
 (segment (start 107.436827 63.063173) (end 110.436827 63.063173) (width 0.5) (layer B.Cu) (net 3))
 (segment (start 110.436827 63.063173) (end 112 61.5) (width 0.5) (layer B.Cu) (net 3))
 (segment (start 111.8 61.3) (end 112 61.5) (width 0.5) (layer F.Cu) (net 3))
 (segment (start 110 61.3) (end 111.8 61.3) (width 0.5) (layer F.Cu) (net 3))
 (via (at 105.5 57) (size 0.8) (drill 0.4) (layers F.Cu B.Cu) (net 1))
 (segment (start 105.5 58.7) (end 105.5 57) (width 0.5) (layer F.Cu) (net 1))
 (via (at 110 57) (size 0.8) (drill 0.4) (layers F.Cu B.Cu) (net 1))
 (segment (start 110 58.7) (end 110 57) (width 0.5) (layer F.Cu) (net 1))
 (segment (start 106.18 74.57) (end 106.18 70.82) (width 0.5) (layer F.Cu) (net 6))
 (segment (start 104.5 76.25) (end 106.18 74.57) (width 0.5) (layer F.Cu) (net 6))
 (segment (start 124.1 64.4) (end 124.1 61.5) (width 0.5) (layer F.Cu) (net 6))
 (segment (start 110.5 66.5) (end 122 66.5) (width 0.5) (layer F.Cu) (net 6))
 (segment (start 106.18 70.82) (end 110.5 66.5) (width 0.5) (layer F.Cu) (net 6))
 (segment (start 122 66.5) (end 124.1 64.4) (width 0.5) (layer F.Cu) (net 6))
 (segment (start 120.54 116) (end 115.46 116) (width 0.5) (layer F.Cu) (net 5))
 (segment (start 108 116) (end 115.46 116) (width 0.5) (layer F.Cu) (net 5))
 (segment (start 102.5 105.78934) (end 102.5 110.5) (width 0.5) (layer F.Cu) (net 5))
 (segment (start 104.5 104.85) (end 103.43934 104.85) (width 0.5) (layer F.Cu) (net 5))
 (segment (start 102.5 110.5) (end 108 116) (width 0.5) (layer F.Cu) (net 5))
 (segment (start 103.43934 104.85) (end 102.5 105.78934) (width 0.5) (layer F.Cu) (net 5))
 (segment (start 117.2 61.5) (end 118.6 61.5) (width 0.5) (layer F.Cu) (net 2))
 (segment (start 115.2 63.5) (end 117.2 61.5) (width 0.5) (layer F.Cu) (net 2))
 (segment (start 106.75 60) (end 107.5 60.75) (width 0.5) (layer F.Cu) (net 2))
 (segment (start 107.5 60.75) (end 107.5 61.5) (width 0.5) (layer F.Cu) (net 2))
 (segment (start 109.5 63.5) (end 115.2 63.5) (width 0.5) (layer F.Cu) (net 2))
 (segment (start 105.5 60) (end 106.75 60) (width 0.5) (layer F.Cu) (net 2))
 (segment (start 107.5 61.5) (end 109.5 63.5) (width 0.5) (layer F.Cu) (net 2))
 (segment (start 116.5 57) (end 113.5 60) (width 0.5) (layer F.Cu) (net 4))
 (segment (start 124.5 57) (end 116.5 57) (width 0.5) (layer F.Cu) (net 4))
 (segment (start 113.5 60) (end 110 60) (width 0.5) (layer F.Cu) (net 4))
 (segment (start 126.5 59) (end 124.5 57) (width 0.5) (layer F.Cu) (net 4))
 (segment (start 126.5 59.5) (end 126.5 59) (width 0.5) (layer F.Cu) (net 4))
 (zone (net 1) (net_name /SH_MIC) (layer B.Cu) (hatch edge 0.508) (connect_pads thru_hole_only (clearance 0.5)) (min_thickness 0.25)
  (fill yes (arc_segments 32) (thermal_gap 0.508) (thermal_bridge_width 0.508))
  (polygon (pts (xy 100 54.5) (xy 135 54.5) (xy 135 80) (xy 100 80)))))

